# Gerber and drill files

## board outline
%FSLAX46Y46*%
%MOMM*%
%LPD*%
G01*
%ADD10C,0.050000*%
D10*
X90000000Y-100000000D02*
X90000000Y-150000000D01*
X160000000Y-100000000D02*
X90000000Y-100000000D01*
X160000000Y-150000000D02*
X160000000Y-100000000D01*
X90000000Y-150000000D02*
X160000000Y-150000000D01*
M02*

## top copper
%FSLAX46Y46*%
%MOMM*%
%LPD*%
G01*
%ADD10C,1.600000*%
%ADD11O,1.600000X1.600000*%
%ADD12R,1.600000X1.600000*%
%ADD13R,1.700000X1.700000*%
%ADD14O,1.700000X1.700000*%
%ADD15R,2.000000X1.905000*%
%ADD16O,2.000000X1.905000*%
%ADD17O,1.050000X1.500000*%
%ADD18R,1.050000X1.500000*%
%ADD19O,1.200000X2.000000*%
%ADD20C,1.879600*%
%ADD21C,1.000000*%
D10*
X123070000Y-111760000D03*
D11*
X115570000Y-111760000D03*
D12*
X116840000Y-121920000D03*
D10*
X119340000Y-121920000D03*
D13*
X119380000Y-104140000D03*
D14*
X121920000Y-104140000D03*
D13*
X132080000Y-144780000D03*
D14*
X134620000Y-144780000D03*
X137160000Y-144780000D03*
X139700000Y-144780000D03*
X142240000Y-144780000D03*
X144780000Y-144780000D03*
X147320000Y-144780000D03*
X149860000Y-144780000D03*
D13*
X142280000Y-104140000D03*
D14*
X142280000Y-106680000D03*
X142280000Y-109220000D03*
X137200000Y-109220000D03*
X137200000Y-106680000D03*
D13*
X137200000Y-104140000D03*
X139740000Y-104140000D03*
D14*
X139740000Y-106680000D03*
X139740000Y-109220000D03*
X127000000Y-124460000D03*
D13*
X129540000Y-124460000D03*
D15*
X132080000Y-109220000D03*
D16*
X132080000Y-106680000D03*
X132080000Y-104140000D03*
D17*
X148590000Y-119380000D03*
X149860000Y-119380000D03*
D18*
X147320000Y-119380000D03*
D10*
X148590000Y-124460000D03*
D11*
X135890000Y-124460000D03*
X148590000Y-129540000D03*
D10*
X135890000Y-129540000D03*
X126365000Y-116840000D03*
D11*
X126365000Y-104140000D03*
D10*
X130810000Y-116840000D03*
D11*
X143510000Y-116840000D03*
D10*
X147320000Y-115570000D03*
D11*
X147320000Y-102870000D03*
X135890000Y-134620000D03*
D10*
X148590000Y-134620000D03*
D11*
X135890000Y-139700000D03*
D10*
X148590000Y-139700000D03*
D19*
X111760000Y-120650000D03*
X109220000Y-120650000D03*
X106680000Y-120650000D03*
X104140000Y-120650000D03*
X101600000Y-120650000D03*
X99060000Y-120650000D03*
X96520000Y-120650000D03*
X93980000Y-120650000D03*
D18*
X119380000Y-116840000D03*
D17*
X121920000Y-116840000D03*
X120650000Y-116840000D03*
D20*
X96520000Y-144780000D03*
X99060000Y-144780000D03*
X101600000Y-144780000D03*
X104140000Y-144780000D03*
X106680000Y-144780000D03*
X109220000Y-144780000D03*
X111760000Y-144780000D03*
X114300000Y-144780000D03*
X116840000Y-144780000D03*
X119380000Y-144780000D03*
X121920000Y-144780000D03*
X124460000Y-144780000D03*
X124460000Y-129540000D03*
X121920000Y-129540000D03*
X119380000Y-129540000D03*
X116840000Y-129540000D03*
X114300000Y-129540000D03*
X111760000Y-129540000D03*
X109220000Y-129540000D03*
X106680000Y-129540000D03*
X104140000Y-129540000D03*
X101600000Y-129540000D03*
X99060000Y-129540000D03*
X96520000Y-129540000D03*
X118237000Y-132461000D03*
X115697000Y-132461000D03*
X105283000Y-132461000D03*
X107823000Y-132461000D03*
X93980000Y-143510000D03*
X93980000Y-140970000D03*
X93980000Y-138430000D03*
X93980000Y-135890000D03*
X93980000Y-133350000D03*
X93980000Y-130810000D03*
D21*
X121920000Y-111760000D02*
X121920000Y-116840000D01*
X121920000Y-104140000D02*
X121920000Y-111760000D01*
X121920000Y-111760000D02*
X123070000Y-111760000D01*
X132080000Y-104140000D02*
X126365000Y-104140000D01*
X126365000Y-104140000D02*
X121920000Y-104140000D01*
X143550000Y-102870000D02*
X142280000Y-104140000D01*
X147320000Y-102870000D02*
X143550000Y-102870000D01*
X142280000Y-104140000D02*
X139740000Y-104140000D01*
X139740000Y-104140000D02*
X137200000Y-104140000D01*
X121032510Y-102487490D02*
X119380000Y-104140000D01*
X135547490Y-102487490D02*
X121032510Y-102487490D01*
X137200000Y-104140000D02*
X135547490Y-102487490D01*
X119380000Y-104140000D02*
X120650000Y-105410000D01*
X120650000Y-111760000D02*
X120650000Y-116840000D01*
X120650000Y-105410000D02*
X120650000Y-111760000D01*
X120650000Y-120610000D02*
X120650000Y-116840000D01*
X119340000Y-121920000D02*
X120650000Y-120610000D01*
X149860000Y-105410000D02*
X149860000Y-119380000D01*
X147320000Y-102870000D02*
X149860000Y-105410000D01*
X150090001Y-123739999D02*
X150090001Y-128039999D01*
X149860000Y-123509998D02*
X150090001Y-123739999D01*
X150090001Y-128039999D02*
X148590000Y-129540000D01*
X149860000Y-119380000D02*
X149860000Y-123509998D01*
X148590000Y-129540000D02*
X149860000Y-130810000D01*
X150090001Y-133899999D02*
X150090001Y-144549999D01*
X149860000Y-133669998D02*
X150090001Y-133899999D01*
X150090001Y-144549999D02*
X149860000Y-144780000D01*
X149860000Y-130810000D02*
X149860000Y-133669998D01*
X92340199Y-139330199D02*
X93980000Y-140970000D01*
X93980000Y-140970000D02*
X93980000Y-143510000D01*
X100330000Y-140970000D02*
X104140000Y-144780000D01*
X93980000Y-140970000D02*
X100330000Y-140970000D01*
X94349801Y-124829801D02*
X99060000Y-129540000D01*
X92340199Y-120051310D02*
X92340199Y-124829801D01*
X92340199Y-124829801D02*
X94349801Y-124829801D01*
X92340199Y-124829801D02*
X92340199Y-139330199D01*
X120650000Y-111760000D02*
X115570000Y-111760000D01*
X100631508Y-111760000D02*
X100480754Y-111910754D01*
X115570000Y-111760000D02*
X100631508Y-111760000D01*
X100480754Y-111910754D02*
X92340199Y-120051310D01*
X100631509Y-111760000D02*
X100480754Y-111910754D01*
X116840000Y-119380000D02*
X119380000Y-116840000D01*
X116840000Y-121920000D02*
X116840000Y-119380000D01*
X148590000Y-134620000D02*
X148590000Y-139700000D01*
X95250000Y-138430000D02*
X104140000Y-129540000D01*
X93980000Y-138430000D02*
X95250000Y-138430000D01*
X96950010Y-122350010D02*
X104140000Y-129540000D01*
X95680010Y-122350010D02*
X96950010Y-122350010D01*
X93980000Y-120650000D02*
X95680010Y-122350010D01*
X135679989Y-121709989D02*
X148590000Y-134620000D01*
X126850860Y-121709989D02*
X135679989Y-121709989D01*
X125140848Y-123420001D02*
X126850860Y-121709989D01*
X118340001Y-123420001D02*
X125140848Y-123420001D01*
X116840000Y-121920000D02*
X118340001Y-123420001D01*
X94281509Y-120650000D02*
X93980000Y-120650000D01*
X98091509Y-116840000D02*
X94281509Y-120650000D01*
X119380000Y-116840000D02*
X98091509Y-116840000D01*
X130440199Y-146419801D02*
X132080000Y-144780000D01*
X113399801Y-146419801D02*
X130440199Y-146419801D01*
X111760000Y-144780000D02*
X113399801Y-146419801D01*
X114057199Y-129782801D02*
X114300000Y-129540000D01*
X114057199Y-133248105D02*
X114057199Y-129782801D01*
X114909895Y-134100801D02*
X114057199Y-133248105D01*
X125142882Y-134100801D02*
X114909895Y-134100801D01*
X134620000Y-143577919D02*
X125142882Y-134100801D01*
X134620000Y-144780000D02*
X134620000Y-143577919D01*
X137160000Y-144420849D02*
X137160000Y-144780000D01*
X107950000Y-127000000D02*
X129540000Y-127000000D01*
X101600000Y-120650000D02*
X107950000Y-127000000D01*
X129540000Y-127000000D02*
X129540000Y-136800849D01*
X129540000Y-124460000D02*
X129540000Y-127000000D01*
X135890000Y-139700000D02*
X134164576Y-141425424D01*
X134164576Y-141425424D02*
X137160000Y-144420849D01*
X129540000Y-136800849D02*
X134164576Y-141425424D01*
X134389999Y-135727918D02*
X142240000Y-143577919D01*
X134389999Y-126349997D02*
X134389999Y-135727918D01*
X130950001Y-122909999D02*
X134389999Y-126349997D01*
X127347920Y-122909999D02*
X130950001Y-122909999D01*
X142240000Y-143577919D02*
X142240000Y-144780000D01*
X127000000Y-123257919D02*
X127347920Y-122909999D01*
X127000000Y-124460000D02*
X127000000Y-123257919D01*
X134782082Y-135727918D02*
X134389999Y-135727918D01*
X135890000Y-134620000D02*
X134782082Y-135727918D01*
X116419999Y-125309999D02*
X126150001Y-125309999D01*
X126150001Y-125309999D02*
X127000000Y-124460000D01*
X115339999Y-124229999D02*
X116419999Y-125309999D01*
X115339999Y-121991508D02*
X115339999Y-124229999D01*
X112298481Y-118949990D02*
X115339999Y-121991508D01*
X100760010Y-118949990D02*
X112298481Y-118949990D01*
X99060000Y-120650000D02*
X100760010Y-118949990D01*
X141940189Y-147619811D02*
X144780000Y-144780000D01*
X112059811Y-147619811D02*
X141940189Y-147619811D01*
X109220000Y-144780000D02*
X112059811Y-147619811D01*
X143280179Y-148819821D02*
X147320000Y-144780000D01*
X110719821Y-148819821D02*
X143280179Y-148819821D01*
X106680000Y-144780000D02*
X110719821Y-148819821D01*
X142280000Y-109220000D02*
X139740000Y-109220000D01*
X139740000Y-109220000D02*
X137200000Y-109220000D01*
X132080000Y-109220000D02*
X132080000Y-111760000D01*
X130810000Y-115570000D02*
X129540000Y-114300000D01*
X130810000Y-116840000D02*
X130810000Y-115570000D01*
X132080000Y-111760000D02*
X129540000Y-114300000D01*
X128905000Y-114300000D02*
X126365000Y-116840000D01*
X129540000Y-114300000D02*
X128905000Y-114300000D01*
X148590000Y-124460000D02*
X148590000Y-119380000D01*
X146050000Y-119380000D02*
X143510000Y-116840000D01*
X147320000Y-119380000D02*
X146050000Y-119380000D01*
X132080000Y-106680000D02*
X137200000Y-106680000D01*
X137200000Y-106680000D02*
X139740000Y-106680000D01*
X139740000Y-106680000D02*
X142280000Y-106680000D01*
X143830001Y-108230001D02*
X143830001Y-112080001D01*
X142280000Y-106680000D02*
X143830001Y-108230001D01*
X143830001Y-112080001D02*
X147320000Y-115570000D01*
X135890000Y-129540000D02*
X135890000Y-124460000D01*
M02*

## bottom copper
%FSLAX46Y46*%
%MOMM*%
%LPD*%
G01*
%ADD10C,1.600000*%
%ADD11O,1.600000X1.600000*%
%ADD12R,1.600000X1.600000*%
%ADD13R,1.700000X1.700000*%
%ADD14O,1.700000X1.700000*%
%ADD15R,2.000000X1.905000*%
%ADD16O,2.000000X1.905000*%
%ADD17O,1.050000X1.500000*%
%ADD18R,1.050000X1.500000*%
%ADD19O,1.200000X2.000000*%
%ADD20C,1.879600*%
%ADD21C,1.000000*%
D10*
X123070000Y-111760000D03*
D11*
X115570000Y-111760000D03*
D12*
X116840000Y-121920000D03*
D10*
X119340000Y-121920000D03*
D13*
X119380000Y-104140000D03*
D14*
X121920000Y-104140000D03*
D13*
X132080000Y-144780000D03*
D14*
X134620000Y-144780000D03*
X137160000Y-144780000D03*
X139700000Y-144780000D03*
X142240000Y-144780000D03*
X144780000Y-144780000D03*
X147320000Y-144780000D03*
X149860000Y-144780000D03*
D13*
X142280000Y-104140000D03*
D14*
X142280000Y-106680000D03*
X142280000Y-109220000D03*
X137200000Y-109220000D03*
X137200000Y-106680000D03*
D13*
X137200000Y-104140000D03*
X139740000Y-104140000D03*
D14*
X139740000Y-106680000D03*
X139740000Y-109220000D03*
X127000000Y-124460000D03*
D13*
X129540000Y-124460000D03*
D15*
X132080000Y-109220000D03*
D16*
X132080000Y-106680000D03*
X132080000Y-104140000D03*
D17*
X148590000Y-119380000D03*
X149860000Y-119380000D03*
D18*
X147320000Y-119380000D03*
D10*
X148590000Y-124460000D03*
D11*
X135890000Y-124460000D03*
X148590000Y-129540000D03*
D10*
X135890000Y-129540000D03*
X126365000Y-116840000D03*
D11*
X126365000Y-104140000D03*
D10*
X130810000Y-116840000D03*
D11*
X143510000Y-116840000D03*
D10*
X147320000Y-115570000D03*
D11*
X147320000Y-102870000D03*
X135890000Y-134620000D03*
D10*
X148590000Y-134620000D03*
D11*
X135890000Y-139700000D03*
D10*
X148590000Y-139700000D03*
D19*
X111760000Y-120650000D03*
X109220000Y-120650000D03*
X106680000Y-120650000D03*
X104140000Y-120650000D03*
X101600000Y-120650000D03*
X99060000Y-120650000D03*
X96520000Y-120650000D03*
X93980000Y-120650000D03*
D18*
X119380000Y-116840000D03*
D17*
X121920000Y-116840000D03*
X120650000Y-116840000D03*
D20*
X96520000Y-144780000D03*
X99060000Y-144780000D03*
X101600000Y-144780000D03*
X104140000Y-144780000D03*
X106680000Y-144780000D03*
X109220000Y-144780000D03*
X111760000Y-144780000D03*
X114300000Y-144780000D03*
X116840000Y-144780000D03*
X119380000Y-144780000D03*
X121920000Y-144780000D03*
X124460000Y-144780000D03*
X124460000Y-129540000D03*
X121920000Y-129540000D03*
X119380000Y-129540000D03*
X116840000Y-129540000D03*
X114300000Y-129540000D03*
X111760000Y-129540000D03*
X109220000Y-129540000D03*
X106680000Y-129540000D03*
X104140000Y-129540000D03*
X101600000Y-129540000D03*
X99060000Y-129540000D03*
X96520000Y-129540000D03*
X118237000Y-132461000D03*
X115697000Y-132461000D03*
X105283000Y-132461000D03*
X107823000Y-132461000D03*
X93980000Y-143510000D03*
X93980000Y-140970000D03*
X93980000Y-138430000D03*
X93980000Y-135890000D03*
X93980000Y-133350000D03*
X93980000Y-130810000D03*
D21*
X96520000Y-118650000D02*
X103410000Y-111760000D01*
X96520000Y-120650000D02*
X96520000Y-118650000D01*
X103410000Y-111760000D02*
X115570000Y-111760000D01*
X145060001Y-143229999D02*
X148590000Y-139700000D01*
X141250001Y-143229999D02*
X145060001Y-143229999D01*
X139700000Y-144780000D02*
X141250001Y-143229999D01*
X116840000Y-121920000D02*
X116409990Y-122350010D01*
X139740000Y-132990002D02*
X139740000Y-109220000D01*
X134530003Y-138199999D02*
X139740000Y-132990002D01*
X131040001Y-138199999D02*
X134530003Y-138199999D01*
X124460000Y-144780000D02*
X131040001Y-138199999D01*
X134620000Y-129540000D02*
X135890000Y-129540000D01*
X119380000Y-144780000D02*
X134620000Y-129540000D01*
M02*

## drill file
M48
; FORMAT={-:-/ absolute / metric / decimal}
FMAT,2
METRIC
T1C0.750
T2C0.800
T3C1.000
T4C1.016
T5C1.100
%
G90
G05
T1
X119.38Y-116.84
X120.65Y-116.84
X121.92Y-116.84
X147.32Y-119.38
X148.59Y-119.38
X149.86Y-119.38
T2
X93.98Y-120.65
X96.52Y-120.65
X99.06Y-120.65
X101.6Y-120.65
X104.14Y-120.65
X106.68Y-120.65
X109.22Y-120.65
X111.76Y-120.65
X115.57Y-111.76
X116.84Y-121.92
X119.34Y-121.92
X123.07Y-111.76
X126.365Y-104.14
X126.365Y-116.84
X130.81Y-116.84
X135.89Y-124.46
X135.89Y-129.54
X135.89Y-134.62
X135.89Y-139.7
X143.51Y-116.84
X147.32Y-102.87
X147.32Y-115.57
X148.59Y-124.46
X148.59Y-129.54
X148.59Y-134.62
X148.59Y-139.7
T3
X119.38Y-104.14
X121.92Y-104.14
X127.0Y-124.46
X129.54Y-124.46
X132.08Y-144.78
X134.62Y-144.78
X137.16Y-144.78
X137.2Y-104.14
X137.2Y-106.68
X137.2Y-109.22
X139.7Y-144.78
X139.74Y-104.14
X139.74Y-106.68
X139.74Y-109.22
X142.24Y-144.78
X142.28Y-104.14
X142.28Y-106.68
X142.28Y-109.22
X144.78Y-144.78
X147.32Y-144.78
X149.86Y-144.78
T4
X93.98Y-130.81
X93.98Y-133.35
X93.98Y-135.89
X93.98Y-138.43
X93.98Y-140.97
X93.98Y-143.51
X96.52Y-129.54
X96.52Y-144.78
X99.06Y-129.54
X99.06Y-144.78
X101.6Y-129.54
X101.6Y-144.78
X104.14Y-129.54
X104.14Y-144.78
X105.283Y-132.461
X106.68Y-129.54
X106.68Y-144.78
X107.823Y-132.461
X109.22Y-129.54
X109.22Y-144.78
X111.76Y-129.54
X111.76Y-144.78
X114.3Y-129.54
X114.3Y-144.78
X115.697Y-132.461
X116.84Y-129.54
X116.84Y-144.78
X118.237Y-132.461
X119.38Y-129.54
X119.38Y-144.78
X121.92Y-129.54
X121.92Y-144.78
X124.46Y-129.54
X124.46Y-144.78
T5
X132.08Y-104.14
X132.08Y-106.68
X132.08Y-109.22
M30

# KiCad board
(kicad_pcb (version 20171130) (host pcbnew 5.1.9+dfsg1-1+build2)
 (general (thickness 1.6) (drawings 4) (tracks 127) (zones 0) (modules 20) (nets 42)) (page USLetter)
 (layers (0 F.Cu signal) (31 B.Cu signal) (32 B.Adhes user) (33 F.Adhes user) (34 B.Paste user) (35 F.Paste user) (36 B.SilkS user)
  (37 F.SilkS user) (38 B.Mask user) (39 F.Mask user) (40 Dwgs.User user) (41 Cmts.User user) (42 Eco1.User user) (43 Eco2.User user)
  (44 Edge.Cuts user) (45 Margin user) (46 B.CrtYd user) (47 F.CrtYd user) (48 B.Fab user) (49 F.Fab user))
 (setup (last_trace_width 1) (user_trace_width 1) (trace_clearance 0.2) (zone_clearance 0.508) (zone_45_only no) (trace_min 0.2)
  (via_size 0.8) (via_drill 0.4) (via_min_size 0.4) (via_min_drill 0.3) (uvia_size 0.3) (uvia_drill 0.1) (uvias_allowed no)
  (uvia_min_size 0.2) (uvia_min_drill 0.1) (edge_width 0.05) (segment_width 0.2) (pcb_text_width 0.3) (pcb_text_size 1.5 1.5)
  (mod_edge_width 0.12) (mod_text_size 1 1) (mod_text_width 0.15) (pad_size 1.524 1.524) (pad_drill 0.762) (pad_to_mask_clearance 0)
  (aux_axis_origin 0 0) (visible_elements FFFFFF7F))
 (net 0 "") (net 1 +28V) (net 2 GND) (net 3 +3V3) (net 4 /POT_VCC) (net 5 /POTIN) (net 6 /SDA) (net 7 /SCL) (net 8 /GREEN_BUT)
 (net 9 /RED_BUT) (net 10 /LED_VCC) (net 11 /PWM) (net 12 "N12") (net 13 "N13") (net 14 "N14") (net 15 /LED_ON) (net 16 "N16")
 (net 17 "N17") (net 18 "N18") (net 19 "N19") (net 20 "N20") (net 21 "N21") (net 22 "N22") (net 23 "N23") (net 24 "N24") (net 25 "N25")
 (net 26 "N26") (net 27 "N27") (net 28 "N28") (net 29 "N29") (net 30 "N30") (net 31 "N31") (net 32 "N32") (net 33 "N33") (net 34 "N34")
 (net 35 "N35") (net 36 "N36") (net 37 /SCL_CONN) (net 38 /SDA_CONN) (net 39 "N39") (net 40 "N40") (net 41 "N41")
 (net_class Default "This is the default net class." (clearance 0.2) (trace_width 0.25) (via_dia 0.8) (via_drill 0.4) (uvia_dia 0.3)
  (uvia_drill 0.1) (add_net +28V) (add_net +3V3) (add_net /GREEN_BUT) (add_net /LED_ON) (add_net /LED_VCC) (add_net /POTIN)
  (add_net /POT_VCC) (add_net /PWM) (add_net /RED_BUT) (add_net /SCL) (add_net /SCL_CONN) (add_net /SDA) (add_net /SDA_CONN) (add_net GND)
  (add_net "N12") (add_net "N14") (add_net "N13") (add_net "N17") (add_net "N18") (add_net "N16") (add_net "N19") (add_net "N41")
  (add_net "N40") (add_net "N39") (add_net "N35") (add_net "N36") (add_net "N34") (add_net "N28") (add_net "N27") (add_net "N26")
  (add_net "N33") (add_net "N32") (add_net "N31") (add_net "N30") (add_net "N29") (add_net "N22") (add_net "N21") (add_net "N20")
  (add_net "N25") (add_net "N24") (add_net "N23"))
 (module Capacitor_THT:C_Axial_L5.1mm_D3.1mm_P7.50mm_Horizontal (layer F.Cu) (at 123.07 111.76 180)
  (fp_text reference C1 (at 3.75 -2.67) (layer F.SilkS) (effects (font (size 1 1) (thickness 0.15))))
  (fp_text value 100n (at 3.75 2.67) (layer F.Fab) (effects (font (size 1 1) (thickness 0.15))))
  (pad 1 thru_hole circle (at 0 0 180) (size 1.6 1.6) (drill 0.8) (layers *.Cu *.Mask) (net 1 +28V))
  (pad 2 thru_hole oval (at 7.5 0 180) (size 1.6 1.6) (drill 0.8) (layers *.Cu *.Mask) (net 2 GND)))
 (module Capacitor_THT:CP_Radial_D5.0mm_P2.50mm (layer F.Cu) (at 116.84 121.92)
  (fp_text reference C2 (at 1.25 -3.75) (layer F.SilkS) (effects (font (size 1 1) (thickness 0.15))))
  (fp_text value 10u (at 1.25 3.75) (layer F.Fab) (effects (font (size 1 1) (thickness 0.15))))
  (pad 1 thru_hole rect (at 0 0) (size 1.6 1.6) (drill 0.8) (layers *.Cu *.Mask) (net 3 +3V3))
  (pad 2 thru_hole circle (at 2.5 0) (size 1.6 1.6) (drill 0.8) (layers *.Cu *.Mask) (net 2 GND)))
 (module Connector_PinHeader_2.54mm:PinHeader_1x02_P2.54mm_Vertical (layer F.Cu) (at 119.38 104.14 90)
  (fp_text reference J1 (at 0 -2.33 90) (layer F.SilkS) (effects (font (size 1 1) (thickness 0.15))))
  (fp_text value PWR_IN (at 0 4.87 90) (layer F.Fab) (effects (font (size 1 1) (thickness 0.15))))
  (pad 1 thru_hole rect (at 0 0 90) (size 1.7 1.7) (drill 1) (layers *.Cu *.Mask) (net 2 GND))
  (pad 2 thru_hole oval (at 0 2.54 90) (size 1.7 1.7) (drill 1) (layers *.Cu *.Mask) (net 1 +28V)))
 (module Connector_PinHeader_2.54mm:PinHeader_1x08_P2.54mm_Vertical (layer F.Cu) (at 132.08 144.78 90)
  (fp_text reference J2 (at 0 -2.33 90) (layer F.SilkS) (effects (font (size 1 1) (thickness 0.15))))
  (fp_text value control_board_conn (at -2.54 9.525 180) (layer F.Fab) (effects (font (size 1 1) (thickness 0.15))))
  (pad 1 thru_hole rect (at 0 0 90) (size 1.7 1.7) (drill 1) (layers *.Cu *.Mask) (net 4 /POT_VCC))
  (pad 2 thru_hole oval (at 0 2.54 90) (size 1.7 1.7) (drill 1) (layers *.Cu *.Mask) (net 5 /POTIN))
  (pad 3 thru_hole oval (at 0 5.08 90) (size 1.7 1.7) (drill 1) (layers *.Cu *.Mask) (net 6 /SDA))
  (pad 4 thru_hole oval (at 0 7.62 90) (size 1.7 1.7) (drill 1) (layers *.Cu *.Mask) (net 3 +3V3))
  (pad 5 thru_hole oval (at 0 10.16 90) (size 1.7 1.7) (drill 1) (layers *.Cu *.Mask) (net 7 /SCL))
  (pad 6 thru_hole oval (at 0 12.7 90) (size 1.7 1.7) (drill 1) (layers *.Cu *.Mask) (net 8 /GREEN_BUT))
  (pad 7 thru_hole oval (at 0 15.24 90) (size 1.7 1.7) (drill 1) (layers *.Cu *.Mask) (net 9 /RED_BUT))
  (pad 8 thru_hole oval (at 0 17.78 90) (size 1.7 1.7) (drill 1) (layers *.Cu *.Mask) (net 2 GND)))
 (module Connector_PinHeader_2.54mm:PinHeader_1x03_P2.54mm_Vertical (layer F.Cu) (at 142.28 104.14)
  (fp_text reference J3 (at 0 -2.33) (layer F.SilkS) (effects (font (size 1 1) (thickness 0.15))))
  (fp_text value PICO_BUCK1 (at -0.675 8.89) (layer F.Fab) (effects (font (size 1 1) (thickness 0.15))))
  (pad 1 thru_hole rect (at 0 0) (size 1.7 1.7) (drill 1) (layers *.Cu *.Mask) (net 2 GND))
  (pad 2 thru_hole oval (at 0 2.54) (size 1.7 1.7) (drill 1) (layers *.Cu *.Mask) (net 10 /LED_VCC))
  (pad 3 thru_hole oval (at 0 5.08) (size 1.7 1.7) (drill 1) (layers *.Cu *.Mask) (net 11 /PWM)))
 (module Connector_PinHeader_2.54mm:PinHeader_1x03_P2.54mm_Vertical (layer F.Cu) (at 137.2 104.14)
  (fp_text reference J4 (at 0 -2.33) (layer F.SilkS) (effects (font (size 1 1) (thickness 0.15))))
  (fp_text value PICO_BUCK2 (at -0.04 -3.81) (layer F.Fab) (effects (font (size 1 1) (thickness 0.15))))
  (pad 3 thru_hole oval (at 0 5.08) (size 1.7 1.7) (drill 1) (layers *.Cu *.Mask) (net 11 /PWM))
  (pad 2 thru_hole oval (at 0 2.54) (size 1.7 1.7) (drill 1) (layers *.Cu *.Mask) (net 10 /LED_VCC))
  (pad 1 thru_hole rect (at 0 0) (size 1.7 1.7) (drill 1) (layers *.Cu *.Mask) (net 2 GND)))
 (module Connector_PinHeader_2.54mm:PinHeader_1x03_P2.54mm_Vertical (layer F.Cu) (at 139.74 104.14)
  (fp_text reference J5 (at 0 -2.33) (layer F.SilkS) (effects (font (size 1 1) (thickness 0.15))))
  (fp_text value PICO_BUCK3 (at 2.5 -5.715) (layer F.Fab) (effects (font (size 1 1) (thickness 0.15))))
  (pad 1 thru_hole rect (at 0 0) (size 1.7 1.7) (drill 1) (layers *.Cu *.Mask) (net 2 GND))
  (pad 2 thru_hole oval (at 0 2.54) (size 1.7 1.7) (drill 1) (layers *.Cu *.Mask) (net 10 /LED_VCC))
  (pad 3 thru_hole oval (at 0 5.08) (size 1.7 1.7) (drill 1) (layers *.Cu *.Mask) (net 11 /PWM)))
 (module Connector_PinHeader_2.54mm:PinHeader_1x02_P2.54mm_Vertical (layer F.Cu) (at 129.54 124.46 270)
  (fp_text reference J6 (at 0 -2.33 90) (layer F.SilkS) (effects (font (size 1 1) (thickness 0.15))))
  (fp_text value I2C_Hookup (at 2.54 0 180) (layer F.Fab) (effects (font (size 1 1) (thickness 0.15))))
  (pad 2 thru_hole oval (at 0 2.54 270) (size 1.7 1.7) (drill 1) (layers *.Cu *.Mask) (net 7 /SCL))
  (pad 1 thru_hole rect (at 0 0 270) (size 1.7 1.7) (drill 1) (layers *.Cu *.Mask) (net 6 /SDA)))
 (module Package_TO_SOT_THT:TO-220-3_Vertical (layer F.Cu) (at 132.08 109.22 90)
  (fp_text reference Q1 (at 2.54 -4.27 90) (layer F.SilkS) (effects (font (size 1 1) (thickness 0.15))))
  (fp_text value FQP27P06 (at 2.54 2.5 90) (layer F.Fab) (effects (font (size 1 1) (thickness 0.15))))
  (pad 1 thru_hole rect (at 0 0 90) (size 1.905 2) (drill 1.1) (layers *.Cu *.Mask) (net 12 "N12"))
  (pad 2 thru_hole oval (at 2.54 0 90) (size 1.905 2) (drill 1.1) (layers *.Cu *.Mask) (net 10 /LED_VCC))
  (pad 3 thru_hole oval (at 5.08 0 90) (size 1.905 2) (drill 1.1) (layers *.Cu *.Mask) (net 1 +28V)))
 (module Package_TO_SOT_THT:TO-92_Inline (layer F.Cu) (at 147.32 119.38)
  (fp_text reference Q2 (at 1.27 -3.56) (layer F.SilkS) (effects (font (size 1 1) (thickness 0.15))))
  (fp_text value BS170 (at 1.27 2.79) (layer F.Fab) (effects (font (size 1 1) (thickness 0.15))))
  (pad 2 thru_hole oval (at 1.27 0) (size 1.05 1.5) (drill 0.75) (layers *.Cu *.Mask) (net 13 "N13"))
  (pad 3 thru_hole oval (at 2.54 0) (size 1.05 1.5) (drill 0.75) (layers *.Cu *.Mask) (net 2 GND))
  (pad 1 thru_hole rect (at 0 0) (size 1.05 1.5) (drill 0.75) (layers *.Cu *.Mask) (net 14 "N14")))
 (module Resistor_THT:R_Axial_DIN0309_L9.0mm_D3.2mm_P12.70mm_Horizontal (layer F.Cu) (at 148.59 124.46 180)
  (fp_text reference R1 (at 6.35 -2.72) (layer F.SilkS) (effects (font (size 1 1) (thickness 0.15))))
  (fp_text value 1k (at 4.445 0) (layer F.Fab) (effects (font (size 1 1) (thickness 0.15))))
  (pad 1 thru_hole circle (at 0 0 180) (size 1.6 1.6) (drill 0.8) (layers *.Cu *.Mask) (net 13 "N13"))
  (pad 2 thru_hole oval (at 12.7 0 180) (size 1.6 1.6) (drill 0.8) (layers *.Cu *.Mask) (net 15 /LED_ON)))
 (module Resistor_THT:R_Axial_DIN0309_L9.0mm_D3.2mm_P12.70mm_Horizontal (layer F.Cu) (at 135.89 129.54)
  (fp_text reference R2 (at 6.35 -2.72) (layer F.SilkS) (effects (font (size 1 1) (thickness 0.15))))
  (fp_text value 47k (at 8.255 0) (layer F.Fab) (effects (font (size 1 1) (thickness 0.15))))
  (pad 2 thru_hole oval (at 12.7 0) (size 1.6 1.6) (drill 0.8) (layers *.Cu *.Mask) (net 2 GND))
  (pad 1 thru_hole circle (at 0 0) (size 1.6 1.6) (drill 0.8) (layers *.Cu *.Mask) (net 15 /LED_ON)))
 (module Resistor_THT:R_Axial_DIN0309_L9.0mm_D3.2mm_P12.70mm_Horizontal (layer F.Cu) (at 126.365 116.84 90)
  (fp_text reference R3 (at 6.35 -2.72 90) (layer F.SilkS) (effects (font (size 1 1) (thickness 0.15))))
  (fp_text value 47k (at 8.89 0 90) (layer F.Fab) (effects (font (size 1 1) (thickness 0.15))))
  (pad 1 thru_hole circle (at 0 0 90) (size 1.6 1.6) (drill 0.8) (layers *.Cu *.Mask) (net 12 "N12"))
  (pad 2 thru_hole oval (at 12.7 0 90) (size 1.6 1.6) (drill 0.8) (layers *.Cu *.Mask) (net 1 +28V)))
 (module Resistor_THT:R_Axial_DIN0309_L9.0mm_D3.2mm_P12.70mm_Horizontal (layer F.Cu) (at 130.81 116.84)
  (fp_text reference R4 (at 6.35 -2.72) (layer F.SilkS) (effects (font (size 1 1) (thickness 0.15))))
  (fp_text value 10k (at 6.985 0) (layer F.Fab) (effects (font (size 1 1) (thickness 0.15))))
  (pad 1 thru_hole circle (at 0 0) (size 1.6 1.6) (drill 0.8) (layers *.Cu *.Mask) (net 12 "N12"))
  (pad 2 thru_hole oval (at 12.7 0) (size 1.6 1.6) (drill 0.8) (layers *.Cu *.Mask) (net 14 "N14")))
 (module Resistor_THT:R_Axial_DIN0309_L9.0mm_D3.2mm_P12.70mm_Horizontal (layer F.Cu) (at 147.32 115.57 90)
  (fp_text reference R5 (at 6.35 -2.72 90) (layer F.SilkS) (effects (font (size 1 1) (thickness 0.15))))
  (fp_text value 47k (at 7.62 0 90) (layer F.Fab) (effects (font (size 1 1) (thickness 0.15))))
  (pad 1 thru_hole circle (at 0 0 90) (size 1.6 1.6) (drill 0.8) (layers *.Cu *.Mask) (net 10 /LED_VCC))
  (pad 2 thru_hole oval (at 12.7 0 90) (size 1.6 1.6) (drill 0.8) (layers *.Cu *.Mask) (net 2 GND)))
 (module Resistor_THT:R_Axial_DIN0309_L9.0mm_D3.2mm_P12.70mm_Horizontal (layer F.Cu) (at 148.59 134.62 180)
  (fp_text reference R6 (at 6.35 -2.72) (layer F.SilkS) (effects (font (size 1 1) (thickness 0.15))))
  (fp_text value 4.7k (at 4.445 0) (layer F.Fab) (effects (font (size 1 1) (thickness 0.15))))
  (pad 2 thru_hole oval (at 12.7 0 180) (size 1.6 1.6) (drill 0.8) (layers *.Cu *.Mask) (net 7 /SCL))
  (pad 1 thru_hole circle (at 0 0 180) (size 1.6 1.6) (drill 0.8) (layers *.Cu *.Mask) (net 3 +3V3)))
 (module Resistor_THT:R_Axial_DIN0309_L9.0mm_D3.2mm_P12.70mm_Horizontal (layer F.Cu) (at 148.59 139.7 180)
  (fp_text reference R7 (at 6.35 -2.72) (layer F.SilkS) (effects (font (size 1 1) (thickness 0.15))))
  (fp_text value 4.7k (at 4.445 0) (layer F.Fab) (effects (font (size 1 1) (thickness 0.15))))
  (pad 2 thru_hole oval (at 12.7 0 180) (size 1.6 1.6) (drill 0.8) (layers *.Cu *.Mask) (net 6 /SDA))
  (pad 1 thru_hole circle (at 0 0 180) (size 1.6 1.6) (drill 0.8) (layers *.Cu *.Mask) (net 3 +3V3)))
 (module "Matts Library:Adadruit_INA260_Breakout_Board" (layer F.Cu) (at 102.87 120.65)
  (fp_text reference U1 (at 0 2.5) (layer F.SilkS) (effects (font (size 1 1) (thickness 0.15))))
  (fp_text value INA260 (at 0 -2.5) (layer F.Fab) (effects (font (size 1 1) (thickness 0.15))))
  (pad 14 thru_hole oval (at 8.89 0) (size 1.2 2) (drill 0.8) (layers *.Cu *.Mask) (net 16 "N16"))
  (pad 1 thru_hole oval (at 6.35 0) (size 1.2 2) (drill 0.8) (layers *.Cu *.Mask) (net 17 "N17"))
  (pad 12 thru_hole oval (at 3.81 0) (size 1.2 2) (drill 0.8) (layers *.Cu *.Mask) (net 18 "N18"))
  (pad 7 thru_hole oval (at 1.27 0) (size 1.2 2) (drill 0.8) (layers *.Cu *.Mask) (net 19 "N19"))
  (pad 8 thru_hole oval (at -1.27 0) (size 1.2 2) (drill 0.8) (layers *.Cu *.Mask) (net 6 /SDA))
  (pad 9 thru_hole oval (at -3.81 0) (size 1.2 2) (drill 0.8) (layers *.Cu *.Mask) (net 7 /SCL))
  (pad 6 thru_hole oval (at -6.35 0) (size 1.2 2) (drill 0.8) (layers *.Cu *.Mask) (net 2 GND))
  (pad 10 thru_hole oval (at -8.89 0) (size 1.2 2) (drill 0.8) (layers *.Cu *.Mask) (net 3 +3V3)))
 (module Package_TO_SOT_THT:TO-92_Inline (layer F.Cu) (at 119.38 116.84)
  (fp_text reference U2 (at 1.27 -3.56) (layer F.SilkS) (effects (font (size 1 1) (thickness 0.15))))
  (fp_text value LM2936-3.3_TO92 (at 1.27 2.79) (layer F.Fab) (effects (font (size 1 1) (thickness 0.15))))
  (pad 1 thru_hole rect (at 0 0) (size 1.05 1.5) (drill 0.75) (layers *.Cu *.Mask) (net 3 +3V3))
  (pad 3 thru_hole oval (at 2.54 0) (size 1.05 1.5) (drill 0.75) (layers *.Cu *.Mask) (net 1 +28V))
  (pad 2 thru_hole oval (at 1.27 0) (size 1.05 1.5) (drill 0.75) (layers *.Cu *.Mask) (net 2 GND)))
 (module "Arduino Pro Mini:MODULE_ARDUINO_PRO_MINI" (layer F.Cu) (at 109.22 137.16 90)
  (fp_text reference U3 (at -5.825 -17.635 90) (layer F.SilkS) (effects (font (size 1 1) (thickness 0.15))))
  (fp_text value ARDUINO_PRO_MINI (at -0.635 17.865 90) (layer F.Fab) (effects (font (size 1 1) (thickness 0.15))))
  (pad JP7_12 thru_hole circle (at -7.62 -12.7 90) (size 1.8796 1.8796) (drill 1.016) (layers *.Cu *.Mask) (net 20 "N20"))
  (pad JP7_11 thru_hole circle (at -7.62 -10.16 90) (size 1.8796 1.8796) (drill 1.016) (layers *.Cu *.Mask) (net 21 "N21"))
  (pad JP7_10 thru_hole circle (at -7.62 -7.62 90) (size 1.8796 1.8796) (drill 1.016) (layers *.Cu *.Mask) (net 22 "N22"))
  (pad JP7_9 thru_hole circle (at -7.62 -5.08 90) (size 1.8796 1.8796) (drill 1.016) (layers *.Cu *.Mask) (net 2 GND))
  (pad JP7_8 thru_hole circle (at -7.62 -2.54 90) (size 1.8796 1.8796) (drill 1.016) (layers *.Cu *.Mask) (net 9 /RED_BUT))
  (pad JP7_7 thru_hole circle (at -7.62 0 90) (size 1.8796 1.8796) (drill 1.016) (layers *.Cu *.Mask) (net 8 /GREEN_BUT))
  (pad JP7_6 thru_hole circle (at -7.62 2.54 90) (size 1.8796 1.8796) (drill 1.016) (layers *.Cu *.Mask) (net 4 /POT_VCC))
  (pad JP7_5 thru_hole circle (at -7.62 5.08 90) (size 1.8796 1.8796) (drill 1.016) (layers *.Cu *.Mask) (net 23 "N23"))
  (pad JP7_4 thru_hole circle (at -7.62 7.62 90) (size 1.8796 1.8796) (drill 1.016) (layers *.Cu *.Mask) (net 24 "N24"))
  (pad JP7_3 thru_hole circle (at -7.62 10.16 90) (size 1.8796 1.8796) (drill 1.016) (layers *.Cu *.Mask) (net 15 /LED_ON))
  (pad JP7_2 thru_hole circle (at -7.62 12.7 90) (size 1.8796 1.8796) (drill 1.016) (layers *.Cu *.Mask) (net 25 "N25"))
  (pad JP7_1 thru_hole circle (at -7.62 15.24 90) (size 1.8796 1.8796) (drill 1.016) (layers *.Cu *.Mask) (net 11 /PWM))
  (pad JP6_12 thru_hole circle (at 7.62 15.24 90) (size 1.8796 1.8796) (drill 1.016) (layers *.Cu *.Mask) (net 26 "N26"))
  (pad JP6_11 thru_hole circle (at 7.62 12.7 90) (size 1.8796 1.8796) (drill 1.016) (layers *.Cu *.Mask) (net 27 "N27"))
  (pad JP6_10 thru_hole circle (at 7.62 10.16 90) (size 1.8796 1.8796) (drill 1.016) (layers *.Cu *.Mask) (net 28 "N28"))
  (pad JP6_9 thru_hole circle (at 7.62 7.62 90) (size 1.8796 1.8796) (drill 1.016) (layers *.Cu *.Mask) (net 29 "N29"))
  (pad JP6_8 thru_hole circle (at 7.62 5.08 90) (size 1.8796 1.8796) (drill 1.016) (layers *.Cu *.Mask) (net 5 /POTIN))
  (pad JP6_7 thru_hole circle (at 7.62 2.54 90) (size 1.8796 1.8796) (drill 1.016) (layers *.Cu *.Mask) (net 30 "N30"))
  (pad JP6_6 thru_hole circle (at 7.62 0 90) (size 1.8796 1.8796) (drill 1.016) (layers *.Cu *.Mask) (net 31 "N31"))
  (pad JP6_5 thru_hole circle (at 7.62 -2.54 90) (size 1.8796 1.8796) (drill 1.016) (layers *.Cu *.Mask) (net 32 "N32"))
  (pad JP6_4 thru_hole circle (at 7.62 -5.08 90) (size 1.8796 1.8796) (drill 1.016) (layers *.Cu *.Mask) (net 3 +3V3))
  (pad JP6_3 thru_hole circle (at 7.62 -7.62 90) (size 1.8796 1.8796) (drill 1.016) (layers *.Cu *.Mask) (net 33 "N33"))
  (pad JP6_2 thru_hole circle (at 7.62 -10.16 90) (size 1.8796 1.8796) (drill 1.016) (layers *.Cu *.Mask) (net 2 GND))
  (pad JP6_1 thru_hole circle (at 7.62 -12.7 90) (size 1.8796 1.8796) (drill 1.016) (layers *.Cu *.Mask) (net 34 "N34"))
  (pad JP3_1 thru_hole circle (at 4.699 9.017 90) (size 1.8796 1.8796) (drill 1.016) (layers *.Cu *.Mask) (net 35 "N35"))
  (pad JP3_2 thru_hole circle (at 4.699 6.477 90) (size 1.8796 1.8796) (drill 1.016) (layers *.Cu *.Mask) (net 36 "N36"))
  (pad JP2_2 thru_hole circle (at 4.699 -3.937 90) (size 1.8796 1.8796) (drill 1.016) (layers *.Cu *.Mask) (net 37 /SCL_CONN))
  (pad JP2_1 thru_hole circle (at 4.699 -1.397 90) (size 1.8796 1.8796) (drill 1.016) (layers *.Cu *.Mask) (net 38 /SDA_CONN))
  (pad JP1_6 thru_hole circle (at -6.35 -15.24 90) (size 1.8796 1.8796) (drill 1.016) (layers *.Cu *.Mask) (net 2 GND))
  (pad JP1_5 thru_hole circle (at -3.81 -15.24 90) (size 1.8796 1.8796) (drill 1.016) (layers *.Cu *.Mask) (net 2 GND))
  (pad JP1_4 thru_hole circle (at -1.27 -15.24 90) (size 1.8796 1.8796) (drill 1.016) (layers *.Cu *.Mask) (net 3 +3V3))
  (pad JP1_3 thru_hole circle (at 1.27 -15.24 90) (size 1.8796 1.8796) (drill 1.016) (layers *.Cu *.Mask) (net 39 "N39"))
  (pad JP1_2 thru_hole circle (at 3.81 -15.24 90) (size 1.8796 1.8796) (drill 1.016) (layers *.Cu *.Mask) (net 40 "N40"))
  (pad JP1_1 thru_hole circle (at 6.35 -15.24 90) (size 1.8796 1.8796) (drill 1.016) (layers *.Cu *.Mask) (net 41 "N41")))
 (gr_line (start 90 100) (end 90 150) (layer Edge.Cuts) (width 0.05))
 (gr_line (start 160 100) (end 90 100) (layer Edge.Cuts) (width 0.05))
 (gr_line (start 160 150) (end 160 100) (layer Edge.Cuts) (width 0.05))
 (gr_line (start 90 150) (end 160 150) (layer Edge.Cuts) (width 0.05))
 (segment (start 121.92 111.76) (end 121.92 116.84) (width 1) (layer F.Cu) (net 1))
 (segment (start 121.92 104.14) (end 121.92 111.76) (width 1) (layer F.Cu) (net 1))
 (segment (start 121.92 111.76) (end 123.07 111.76) (width 1) (layer F.Cu) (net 1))
 (segment (start 132.08 104.14) (end 126.365 104.14) (width 1) (layer F.Cu) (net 1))
 (segment (start 126.365 104.14) (end 121.92 104.14) (width 1) (layer F.Cu) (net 1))
 (segment (start 143.55 102.87) (end 142.28 104.14) (width 1) (layer F.Cu) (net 2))
 (segment (start 147.32 102.87) (end 143.55 102.87) (width 1) (layer F.Cu) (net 2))
 (segment (start 142.28 104.14) (end 139.74 104.14) (width 1) (layer F.Cu) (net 2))
 (segment (start 139.74 104.14) (end 137.2 104.14) (width 1) (layer F.Cu) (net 2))
 (segment (start 121.03251 102.48749) (end 119.38 104.14) (width 1) (layer F.Cu) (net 2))
 (segment (start 135.54749 102.48749) (end 121.03251 102.48749) (width 1) (layer F.Cu) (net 2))
 (segment (start 137.2 104.14) (end 135.54749 102.48749) (width 1) (layer F.Cu) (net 2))
 (segment (start 119.38 104.14) (end 120.65 105.41) (width 1) (layer F.Cu) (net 2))
 (segment (start 120.65 111.76) (end 120.65 116.84) (width 1) (layer F.Cu) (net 2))
 (segment (start 120.65 105.41) (end 120.65 111.76) (width 1) (layer F.Cu) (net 2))
 (segment (start 120.65 120.61) (end 120.65 116.84) (width 1) (layer F.Cu) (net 2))
 (segment (start 119.34 121.92) (end 120.65 120.61) (width 1) (layer F.Cu) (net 2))
 (segment (start 149.86 105.41) (end 149.86 119.38) (width 1) (layer F.Cu) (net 2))
 (segment (start 147.32 102.87) (end 149.86 105.41) (width 1) (layer F.Cu) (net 2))
 (segment (start 150.090001 123.739999) (end 150.090001 128.039999) (width 1) (layer F.Cu) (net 2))
 (segment (start 149.86 123.509998) (end 150.090001 123.739999) (width 1) (layer F.Cu) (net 2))
 (segment (start 150.090001 128.039999) (end 148.59 129.54) (width 1) (layer F.Cu) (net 2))
 (segment (start 149.86 119.38) (end 149.86 123.509998) (width 1) (layer F.Cu) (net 2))
 (segment (start 148.59 129.54) (end 149.86 130.81) (width 1) (layer F.Cu) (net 2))
 (segment (start 150.090001 133.899999) (end 150.090001 144.549999) (width 1) (layer F.Cu) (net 2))
 (segment (start 149.86 133.669998) (end 150.090001 133.899999) (width 1) (layer F.Cu) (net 2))
 (segment (start 150.090001 144.549999) (end 149.86 144.78) (width 1) (layer F.Cu) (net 2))
 (segment (start 149.86 130.81) (end 149.86 133.669998) (width 1) (layer F.Cu) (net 2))
 (segment (start 92.340199 139.330199) (end 93.98 140.97) (width 1) (layer F.Cu) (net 2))
 (segment (start 93.98 140.97) (end 93.98 143.51) (width 1) (layer F.Cu) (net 2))
 (segment (start 100.33 140.97) (end 104.14 144.78) (width 1) (layer F.Cu) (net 2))
 (segment (start 93.98 140.97) (end 100.33 140.97) (width 1) (layer F.Cu) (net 2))
 (segment (start 94.349801 124.829801) (end 99.06 129.54) (width 1) (layer F.Cu) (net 2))
 (segment (start 92.340199 120.05131) (end 92.340199 124.829801) (width 1) (layer F.Cu) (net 2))
 (segment (start 92.340199 124.829801) (end 94.349801 124.829801) (width 1) (layer F.Cu) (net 2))
 (segment (start 92.340199 124.829801) (end 92.340199 139.330199) (width 1) (layer F.Cu) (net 2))
 (segment (start 96.52 118.65) (end 103.41 111.76) (width 1) (layer B.Cu) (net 2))
 (segment (start 96.52 120.65) (end 96.52 118.65) (width 1) (layer B.Cu) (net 2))
 (segment (start 120.65 111.76) (end 115.57 111.76) (width 1) (layer F.Cu) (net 2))
 (segment (start 100.631508 111.76) (end 100.480754 111.910754) (width 1) (layer F.Cu) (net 2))
 (segment (start 115.57 111.76) (end 100.631508 111.76) (width 1) (layer F.Cu) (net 2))
 (segment (start 100.480754 111.910754) (end 92.340199 120.05131) (width 1) (layer F.Cu) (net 2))
 (segment (start 100.631509 111.76) (end 100.480754 111.910754) (width 1) (layer F.Cu) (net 2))
 (segment (start 103.41 111.76) (end 115.57 111.76) (width 1) (layer B.Cu) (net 2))
 (segment (start 116.84 119.38) (end 119.38 116.84) (width 1) (layer F.Cu) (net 3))
 (segment (start 116.84 121.92) (end 116.84 119.38) (width 1) (layer F.Cu) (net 3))
 (segment (start 145.060001 143.229999) (end 148.59 139.7) (width 1) (layer B.Cu) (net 3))
 (segment (start 141.250001 143.229999) (end 145.060001 143.229999) (width 1) (layer B.Cu) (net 3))
 (segment (start 139.7 144.78) (end 141.250001 143.229999) (width 1) (layer B.Cu) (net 3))
 (segment (start 148.59 134.62) (end 148.59 139.7) (width 1) (layer F.Cu) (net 3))
 (segment (start 95.25 138.43) (end 104.14 129.54) (width 1) (layer F.Cu) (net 3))
 (segment (start 93.98 138.43) (end 95.25 138.43) (width 1) (layer F.Cu) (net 3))
 (segment (start 96.95001 122.35001) (end 104.14 129.54) (width 1) (layer F.Cu) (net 3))
 (segment (start 95.68001 122.35001) (end 96.95001 122.35001) (width 1) (layer F.Cu) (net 3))
 (segment (start 93.98 120.65) (end 95.68001 122.35001) (width 1) (layer F.Cu) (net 3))
 (segment (start 116.84 121.92) (end 116.40999 122.35001) (width 1) (layer B.Cu) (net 3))
 (segment (start 135.679989 121.709989) (end 148.59 134.62) (width 1) (layer F.Cu) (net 3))
 (segment (start 126.85086 121.709989) (end 135.679989 121.709989) (width 1) (layer F.Cu) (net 3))
 (segment (start 125.140848 123.420001) (end 126.85086 121.709989) (width 1) (layer F.Cu) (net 3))
 (segment (start 118.340001 123.420001) (end 125.140848 123.420001) (width 1) (layer F.Cu) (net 3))
 (segment (start 116.84 121.92) (end 118.340001 123.420001) (width 1) (layer F.Cu) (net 3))
 (segment (start 94.281509 120.65) (end 93.98 120.65) (width 1) (layer F.Cu) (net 3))
 (segment (start 98.091509 116.84) (end 94.281509 120.65) (width 1) (layer F.Cu) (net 3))
 (segment (start 119.38 116.84) (end 98.091509 116.84) (width 1) (layer F.Cu) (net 3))
 (segment (start 130.440199 146.419801) (end 132.08 144.78) (width 1) (layer F.Cu) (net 4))
 (segment (start 113.399801 146.419801) (end 130.440199 146.419801) (width 1) (layer F.Cu) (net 4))
 (segment (start 111.76 144.78) (end 113.399801 146.419801) (width 1) (layer F.Cu) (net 4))
 (segment (start 114.057199 129.782801) (end 114.3 129.54) (width 1) (layer F.Cu) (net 5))
 (segment (start 114.057199 133.248105) (end 114.057199 129.782801) (width 1) (layer F.Cu) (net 5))
 (segment (start 114.909895 134.100801) (end 114.057199 133.248105) (width 1) (layer F.Cu) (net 5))
 (segment (start 125.142882 134.100801) (end 114.909895 134.100801) (width 1) (layer F.Cu) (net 5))
 (segment (start 134.62 143.577919) (end 125.142882 134.100801) (width 1) (layer F.Cu) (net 5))
 (segment (start 134.62 144.78) (end 134.62 143.577919) (width 1) (layer F.Cu) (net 5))
 (segment (start 137.16 144.420849) (end 137.16 144.78) (width 1) (layer F.Cu) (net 6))
 (segment (start 107.95 127) (end 129.54 127) (width 1) (layer F.Cu) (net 6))
 (segment (start 101.6 120.65) (end 107.95 127) (width 1) (layer F.Cu) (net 6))
 (segment (start 129.54 127) (end 129.54 136.800849) (width 1) (layer F.Cu) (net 6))
 (segment (start 129.54 124.46) (end 129.54 127) (width 1) (layer F.Cu) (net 6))
 (segment (start 135.89 139.7) (end 134.164576 141.425424) (width 1) (layer F.Cu) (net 6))
 (segment (start 134.164576 141.425424) (end 137.16 144.420849) (width 1) (layer F.Cu) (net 6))
 (segment (start 129.54 136.800849) (end 134.164576 141.425424) (width 1) (layer F.Cu) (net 6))
 (segment (start 134.389999 135.727918) (end 142.24 143.577919) (width 1) (layer F.Cu) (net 7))
 (segment (start 134.389999 126.349997) (end 134.389999 135.727918) (width 1) (layer F.Cu) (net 7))
 (segment (start 130.950001 122.909999) (end 134.389999 126.349997) (width 1) (layer F.Cu) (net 7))
 (segment (start 127.34792 122.909999) (end 130.950001 122.909999) (width 1) (layer F.Cu) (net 7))
 (segment (start 142.24 143.577919) (end 142.24 144.78) (width 1) (layer F.Cu) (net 7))
 (segment (start 127 123.257919) (end 127.34792 122.909999) (width 1) (layer F.Cu) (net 7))
 (segment (start 127 124.46) (end 127 123.257919) (width 1) (layer F.Cu) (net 7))
 (segment (start 134.782082 135.727918) (end 134.389999 135.727918) (width 1) (layer F.Cu) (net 7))
 (segment (start 135.89 134.62) (end 134.782082 135.727918) (width 1) (layer F.Cu) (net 7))
 (segment (start 116.419999 125.309999) (end 126.150001 125.309999) (width 1) (layer F.Cu) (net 7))
 (segment (start 126.150001 125.309999) (end 127 124.46) (width 1) (layer F.Cu) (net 7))
 (segment (start 115.339999 124.229999) (end 116.419999 125.309999) (width 1) (layer F.Cu) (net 7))
 (segment (start 115.339999 121.991508) (end 115.339999 124.229999) (width 1) (layer F.Cu) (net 7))
 (segment (start 112.298481 118.94999) (end 115.339999 121.991508) (width 1) (layer F.Cu) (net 7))
 (segment (start 100.76001 118.94999) (end 112.298481 118.94999) (width 1) (layer F.Cu) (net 7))
 (segment (start 99.06 120.65) (end 100.76001 118.94999) (width 1) (layer F.Cu) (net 7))
 (segment (start 141.940189 147.619811) (end 144.78 144.78) (width 1) (layer F.Cu) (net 8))
 (segment (start 112.059811 147.619811) (end 141.940189 147.619811) (width 1) (layer F.Cu) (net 8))
 (segment (start 109.22 144.78) (end 112.059811 147.619811) (width 1) (layer F.Cu) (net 8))
 (segment (start 143.280179 148.819821) (end 147.32 144.78) (width 1) (layer F.Cu) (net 9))
 (segment (start 110.719821 148.819821) (end 143.280179 148.819821) (width 1) (layer F.Cu) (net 9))
 (segment (start 106.68 144.78) (end 110.719821 148.819821) (width 1) (layer F.Cu) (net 9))
 (segment (start 142.28 109.22) (end 139.74 109.22) (width 1) (layer F.Cu) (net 11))
 (segment (start 139.74 109.22) (end 137.2 109.22) (width 1) (layer F.Cu) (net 11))
 (segment (start 139.74 132.990002) (end 139.74 109.22) (width 1) (layer B.Cu) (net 11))
 (segment (start 134.530003 138.199999) (end 139.74 132.990002) (width 1) (layer B.Cu) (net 11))
 (segment (start 131.040001 138.199999) (end 134.530003 138.199999) (width 1) (layer B.Cu) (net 11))
 (segment (start 124.46 144.78) (end 131.040001 138.199999) (width 1) (layer B.Cu) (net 11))
 (segment (start 132.08 109.22) (end 132.08 111.76) (width 1) (layer F.Cu) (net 12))
 (segment (start 130.81 115.57) (end 129.54 114.3) (width 1) (layer F.Cu) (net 12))
 (segment (start 130.81 116.84) (end 130.81 115.57) (width 1) (layer F.Cu) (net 12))
 (segment (start 132.08 111.76) (end 129.54 114.3) (width 1) (layer F.Cu) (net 12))
 (segment (start 128.905 114.3) (end 126.365 116.84) (width 1) (layer F.Cu) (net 12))
 (segment (start 129.54 114.3) (end 128.905 114.3) (width 1) (layer F.Cu) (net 12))
 (segment (start 148.59 124.46) (end 148.59 119.38) (width 1) (layer F.Cu) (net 13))
 (segment (start 146.05 119.38) (end 143.51 116.84) (width 1) (layer F.Cu) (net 14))
 (segment (start 147.32 119.38) (end 146.05 119.38) (width 1) (layer F.Cu) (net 14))
 (segment (start 132.08 106.68) (end 137.2 106.68) (width 1) (layer F.Cu) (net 10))
 (segment (start 137.2 106.68) (end 139.74 106.68) (width 1) (layer F.Cu) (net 10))
 (segment (start 139.74 106.68) (end 142.28 106.68) (width 1) (layer F.Cu) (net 10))
 (segment (start 143.830001 108.230001) (end 143.830001 112.080001) (width 1) (layer F.Cu) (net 10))
 (segment (start 142.28 106.68) (end 143.830001 108.230001) (width 1) (layer F.Cu) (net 10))
 (segment (start 143.830001 112.080001) (end 147.32 115.57) (width 1) (layer F.Cu) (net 10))
 (segment (start 134.62 129.54) (end 135.89 129.54) (width 1) (layer B.Cu) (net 15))
 (segment (start 119.38 144.78) (end 134.62 129.54) (width 1) (layer B.Cu) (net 15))
 (segment (start 135.89 129.54) (end 135.89 124.46) (width 1) (layer F.Cu) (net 15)))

